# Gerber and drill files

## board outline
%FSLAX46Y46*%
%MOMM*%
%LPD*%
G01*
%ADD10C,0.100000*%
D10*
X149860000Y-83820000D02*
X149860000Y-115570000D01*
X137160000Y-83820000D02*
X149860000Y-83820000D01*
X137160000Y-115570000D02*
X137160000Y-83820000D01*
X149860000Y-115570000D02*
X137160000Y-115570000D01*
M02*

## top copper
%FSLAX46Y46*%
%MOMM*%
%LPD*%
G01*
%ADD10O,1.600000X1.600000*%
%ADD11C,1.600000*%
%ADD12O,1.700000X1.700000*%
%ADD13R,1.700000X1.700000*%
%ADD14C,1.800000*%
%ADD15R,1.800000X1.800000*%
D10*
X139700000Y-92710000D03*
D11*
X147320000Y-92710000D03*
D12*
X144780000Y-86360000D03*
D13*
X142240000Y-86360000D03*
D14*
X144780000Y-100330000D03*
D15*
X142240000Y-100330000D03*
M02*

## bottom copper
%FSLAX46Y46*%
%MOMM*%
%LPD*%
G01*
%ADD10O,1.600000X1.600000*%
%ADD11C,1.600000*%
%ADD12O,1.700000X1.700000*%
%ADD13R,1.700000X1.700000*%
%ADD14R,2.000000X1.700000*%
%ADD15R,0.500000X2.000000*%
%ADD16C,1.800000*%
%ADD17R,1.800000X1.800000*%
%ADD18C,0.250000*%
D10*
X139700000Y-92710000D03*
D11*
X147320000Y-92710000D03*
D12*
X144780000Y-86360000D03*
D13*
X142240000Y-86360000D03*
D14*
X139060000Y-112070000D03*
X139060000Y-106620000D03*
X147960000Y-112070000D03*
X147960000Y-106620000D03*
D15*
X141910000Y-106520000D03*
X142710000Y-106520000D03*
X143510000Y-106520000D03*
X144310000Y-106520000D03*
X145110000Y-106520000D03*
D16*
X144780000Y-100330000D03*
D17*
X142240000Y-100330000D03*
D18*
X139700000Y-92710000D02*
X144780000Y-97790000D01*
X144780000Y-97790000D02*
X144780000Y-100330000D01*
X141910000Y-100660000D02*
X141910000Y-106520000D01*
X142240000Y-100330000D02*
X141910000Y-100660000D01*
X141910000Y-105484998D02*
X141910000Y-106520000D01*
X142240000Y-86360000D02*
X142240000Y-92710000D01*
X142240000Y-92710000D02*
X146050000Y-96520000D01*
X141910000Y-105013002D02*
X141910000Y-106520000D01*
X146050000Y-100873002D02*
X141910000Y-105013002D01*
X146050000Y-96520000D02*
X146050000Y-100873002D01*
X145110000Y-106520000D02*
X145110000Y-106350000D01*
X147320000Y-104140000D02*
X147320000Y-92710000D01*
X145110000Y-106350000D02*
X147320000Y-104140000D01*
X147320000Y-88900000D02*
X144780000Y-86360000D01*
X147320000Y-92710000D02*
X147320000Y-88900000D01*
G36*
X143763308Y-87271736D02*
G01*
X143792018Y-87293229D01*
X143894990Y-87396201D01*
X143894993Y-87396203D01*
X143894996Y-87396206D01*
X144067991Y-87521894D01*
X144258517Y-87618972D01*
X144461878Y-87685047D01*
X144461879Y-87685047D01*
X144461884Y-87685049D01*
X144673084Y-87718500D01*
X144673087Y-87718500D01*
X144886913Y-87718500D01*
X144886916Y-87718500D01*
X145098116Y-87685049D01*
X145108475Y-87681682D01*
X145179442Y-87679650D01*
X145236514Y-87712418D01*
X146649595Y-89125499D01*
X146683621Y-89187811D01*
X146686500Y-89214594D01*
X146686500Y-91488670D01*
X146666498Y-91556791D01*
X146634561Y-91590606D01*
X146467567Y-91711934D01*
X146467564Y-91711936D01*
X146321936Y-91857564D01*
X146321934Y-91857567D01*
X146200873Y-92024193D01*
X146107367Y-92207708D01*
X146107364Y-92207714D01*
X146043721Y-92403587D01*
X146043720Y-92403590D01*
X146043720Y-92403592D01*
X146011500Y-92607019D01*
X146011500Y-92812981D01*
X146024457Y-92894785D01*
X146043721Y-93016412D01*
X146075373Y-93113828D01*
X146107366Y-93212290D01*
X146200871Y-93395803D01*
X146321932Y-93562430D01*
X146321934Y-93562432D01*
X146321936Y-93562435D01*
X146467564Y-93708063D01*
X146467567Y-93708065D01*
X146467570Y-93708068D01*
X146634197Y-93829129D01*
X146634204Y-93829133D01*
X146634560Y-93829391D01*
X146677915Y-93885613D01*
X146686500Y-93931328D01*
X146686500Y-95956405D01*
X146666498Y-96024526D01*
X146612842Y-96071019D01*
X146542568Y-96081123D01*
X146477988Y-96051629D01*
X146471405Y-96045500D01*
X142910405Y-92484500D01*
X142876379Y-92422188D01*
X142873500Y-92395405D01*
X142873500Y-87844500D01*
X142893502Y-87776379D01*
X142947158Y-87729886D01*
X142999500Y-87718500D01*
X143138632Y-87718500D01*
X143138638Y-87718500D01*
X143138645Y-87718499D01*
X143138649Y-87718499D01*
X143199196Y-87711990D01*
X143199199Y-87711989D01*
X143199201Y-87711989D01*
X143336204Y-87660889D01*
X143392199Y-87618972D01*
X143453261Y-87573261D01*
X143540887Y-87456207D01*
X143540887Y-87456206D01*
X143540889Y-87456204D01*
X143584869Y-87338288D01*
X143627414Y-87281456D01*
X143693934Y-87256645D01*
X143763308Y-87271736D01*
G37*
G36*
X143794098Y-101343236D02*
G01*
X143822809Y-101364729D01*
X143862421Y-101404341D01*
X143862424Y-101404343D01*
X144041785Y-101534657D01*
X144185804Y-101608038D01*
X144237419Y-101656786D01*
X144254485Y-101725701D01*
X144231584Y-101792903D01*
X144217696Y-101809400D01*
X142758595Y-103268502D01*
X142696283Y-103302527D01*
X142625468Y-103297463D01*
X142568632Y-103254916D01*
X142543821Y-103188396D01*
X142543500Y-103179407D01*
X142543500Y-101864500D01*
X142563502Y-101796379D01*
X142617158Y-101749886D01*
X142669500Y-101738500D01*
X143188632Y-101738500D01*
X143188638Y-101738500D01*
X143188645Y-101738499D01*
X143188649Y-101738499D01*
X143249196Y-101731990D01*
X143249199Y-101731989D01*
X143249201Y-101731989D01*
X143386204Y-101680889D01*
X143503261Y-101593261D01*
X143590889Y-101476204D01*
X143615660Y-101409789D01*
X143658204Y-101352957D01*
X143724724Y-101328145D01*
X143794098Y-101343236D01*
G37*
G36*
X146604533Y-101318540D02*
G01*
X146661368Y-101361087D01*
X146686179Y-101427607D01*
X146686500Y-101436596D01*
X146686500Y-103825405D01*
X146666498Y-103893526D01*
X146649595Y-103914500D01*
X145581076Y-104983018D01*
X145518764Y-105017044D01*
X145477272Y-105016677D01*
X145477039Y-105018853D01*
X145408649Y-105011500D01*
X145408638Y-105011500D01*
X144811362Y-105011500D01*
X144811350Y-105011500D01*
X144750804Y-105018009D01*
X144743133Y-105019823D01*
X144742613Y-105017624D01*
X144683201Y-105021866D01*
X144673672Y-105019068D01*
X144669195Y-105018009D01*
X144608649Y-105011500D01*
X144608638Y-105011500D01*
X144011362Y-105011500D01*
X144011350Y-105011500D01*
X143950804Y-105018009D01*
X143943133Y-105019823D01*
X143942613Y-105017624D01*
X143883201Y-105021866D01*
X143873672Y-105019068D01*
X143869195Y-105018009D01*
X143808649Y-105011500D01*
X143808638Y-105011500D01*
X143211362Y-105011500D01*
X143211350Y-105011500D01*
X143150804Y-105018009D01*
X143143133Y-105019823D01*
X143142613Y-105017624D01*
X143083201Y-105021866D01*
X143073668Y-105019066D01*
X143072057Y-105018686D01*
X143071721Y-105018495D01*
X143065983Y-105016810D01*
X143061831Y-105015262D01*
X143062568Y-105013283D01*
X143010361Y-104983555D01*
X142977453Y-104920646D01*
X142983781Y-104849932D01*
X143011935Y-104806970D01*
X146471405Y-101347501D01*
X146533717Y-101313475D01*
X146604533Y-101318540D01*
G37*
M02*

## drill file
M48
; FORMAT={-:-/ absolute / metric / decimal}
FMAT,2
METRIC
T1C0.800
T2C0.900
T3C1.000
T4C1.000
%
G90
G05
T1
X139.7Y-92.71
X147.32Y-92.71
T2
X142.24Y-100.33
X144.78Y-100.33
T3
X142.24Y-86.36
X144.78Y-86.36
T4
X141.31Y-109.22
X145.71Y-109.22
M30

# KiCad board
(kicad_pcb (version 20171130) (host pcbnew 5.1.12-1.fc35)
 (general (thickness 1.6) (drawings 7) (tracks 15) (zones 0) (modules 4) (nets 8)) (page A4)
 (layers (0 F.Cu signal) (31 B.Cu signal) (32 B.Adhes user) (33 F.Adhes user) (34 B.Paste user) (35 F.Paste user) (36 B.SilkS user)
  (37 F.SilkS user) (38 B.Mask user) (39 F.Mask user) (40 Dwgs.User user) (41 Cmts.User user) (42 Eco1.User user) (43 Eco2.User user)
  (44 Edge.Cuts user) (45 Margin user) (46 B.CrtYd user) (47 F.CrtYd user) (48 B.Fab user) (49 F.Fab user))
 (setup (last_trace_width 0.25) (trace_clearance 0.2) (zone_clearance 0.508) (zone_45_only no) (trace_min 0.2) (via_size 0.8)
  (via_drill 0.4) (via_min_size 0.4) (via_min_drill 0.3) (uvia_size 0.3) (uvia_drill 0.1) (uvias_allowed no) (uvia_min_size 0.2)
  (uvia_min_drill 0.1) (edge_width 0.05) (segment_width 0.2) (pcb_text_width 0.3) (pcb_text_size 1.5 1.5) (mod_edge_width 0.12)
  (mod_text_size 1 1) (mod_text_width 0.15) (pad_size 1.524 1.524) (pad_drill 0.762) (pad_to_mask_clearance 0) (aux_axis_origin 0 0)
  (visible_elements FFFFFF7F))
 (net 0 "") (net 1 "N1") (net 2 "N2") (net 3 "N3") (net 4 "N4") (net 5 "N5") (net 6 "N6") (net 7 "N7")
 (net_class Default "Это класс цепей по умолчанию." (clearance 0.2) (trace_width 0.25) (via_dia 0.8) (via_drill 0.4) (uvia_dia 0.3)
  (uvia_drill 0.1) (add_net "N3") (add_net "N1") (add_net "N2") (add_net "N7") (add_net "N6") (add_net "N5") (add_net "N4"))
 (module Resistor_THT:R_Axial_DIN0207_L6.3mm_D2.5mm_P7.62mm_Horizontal (layer F.Cu) (at 147.32 92.71 180)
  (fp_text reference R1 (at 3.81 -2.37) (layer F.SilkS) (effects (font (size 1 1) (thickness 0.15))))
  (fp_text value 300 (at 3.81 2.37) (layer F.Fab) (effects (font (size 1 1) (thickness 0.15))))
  (pad 2 thru_hole oval (at 7.62 0 180) (size 1.6 1.6) (drill 0.8) (layers *.Cu *.Mask) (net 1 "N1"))
  (pad 1 thru_hole circle (at 0 0 180) (size 1.6 1.6) (drill 0.8) (layers *.Cu *.Mask) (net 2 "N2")))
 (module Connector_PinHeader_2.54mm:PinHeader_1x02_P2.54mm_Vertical (layer F.Cu) (at 142.24 86.36 90)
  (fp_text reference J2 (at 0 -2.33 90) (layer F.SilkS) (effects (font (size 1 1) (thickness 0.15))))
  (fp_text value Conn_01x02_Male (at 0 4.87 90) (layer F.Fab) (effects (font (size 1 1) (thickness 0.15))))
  (pad 2 thru_hole oval (at 0 2.54 90) (size 1.7 1.7) (drill 1) (layers *.Cu *.Mask) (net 2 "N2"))
  (pad 1 thru_hole rect (at 0 0 90) (size 1.7 1.7) (drill 1) (layers *.Cu *.Mask) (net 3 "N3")))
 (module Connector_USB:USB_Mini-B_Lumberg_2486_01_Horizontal (layer B.Cu) (at 143.51 109.22 180)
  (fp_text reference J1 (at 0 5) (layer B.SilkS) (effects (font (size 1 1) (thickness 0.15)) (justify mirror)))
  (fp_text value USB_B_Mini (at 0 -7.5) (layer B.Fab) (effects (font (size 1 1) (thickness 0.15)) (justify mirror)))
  (pad "" np_thru_hole circle (at 2.2 0 180) (size 1 1) (drill 1) (layers *.Cu *.Mask))
  (pad "" np_thru_hole circle (at -2.2 0 180) (size 1 1) (drill 1) (layers *.Cu *.Mask))
  (pad 6 smd rect (at 4.45 -2.85 180) (size 2 1.7) (layers B.Cu B.Paste B.Mask) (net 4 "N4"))
  (pad 6 smd rect (at 4.45 2.6 180) (size 2 1.7) (layers B.Cu B.Paste B.Mask) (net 4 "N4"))
  (pad 6 smd rect (at -4.45 -2.85 180) (size 2 1.7) (layers B.Cu B.Paste B.Mask) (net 4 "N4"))
  (pad 6 smd rect (at -4.45 2.6 180) (size 2 1.7) (layers B.Cu B.Paste B.Mask) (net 4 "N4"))
  (pad 5 smd rect (at 1.6 2.7 180) (size 0.5 2) (layers B.Cu B.Paste B.Mask) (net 3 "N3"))
  (pad 4 smd rect (at 0.8 2.7 180) (size 0.5 2) (layers B.Cu B.Paste B.Mask) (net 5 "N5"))
  (pad 3 smd rect (at 0 2.7 180) (size 0.5 2) (layers B.Cu B.Paste B.Mask) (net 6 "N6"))
  (pad 2 smd rect (at -0.8 2.7 180) (size 0.5 2) (layers B.Cu B.Paste B.Mask) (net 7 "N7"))
  (pad 1 smd rect (at -1.6 2.7 180) (size 0.5 2) (layers B.Cu B.Paste B.Mask) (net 2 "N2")))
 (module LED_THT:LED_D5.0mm (layer F.Cu) (at 142.24 100.33)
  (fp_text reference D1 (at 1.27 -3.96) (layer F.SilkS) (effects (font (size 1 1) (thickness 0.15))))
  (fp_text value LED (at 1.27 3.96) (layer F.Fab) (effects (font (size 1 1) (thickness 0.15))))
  (pad 2 thru_hole circle (at 2.54 0) (size 1.8 1.8) (drill 0.9) (layers *.Cu *.Mask) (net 1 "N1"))
  (pad 1 thru_hole rect (at 0 0) (size 1.8 1.8) (drill 0.9) (layers *.Cu *.Mask) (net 3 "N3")))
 (gr_line (start 149.86 83.82) (end 149.86 115.57) (layer Edge.Cuts) (width 0.1))
 (gr_line (start 137.16 83.82) (end 149.86 83.82) (layer Edge.Cuts) (width 0.1))
 (gr_line (start 137.16 115.57) (end 137.16 83.82) (layer Edge.Cuts) (width 0.1))
 (gr_line (start 149.86 115.57) (end 137.16 115.57) (layer Edge.Cuts) (width 0.1))
 (segment (start 139.7 92.71) (end 144.78 97.79) (width 0.25) (layer B.Cu) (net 1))
 (segment (start 144.78 97.79) (end 144.78 100.33) (width 0.25) (layer B.Cu) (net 1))
 (segment (start 141.91 100.66) (end 141.91 106.52) (width 0.25) (layer B.Cu) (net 3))
 (segment (start 142.24 100.33) (end 141.91 100.66) (width 0.25) (layer B.Cu) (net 3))
 (segment (start 141.91 105.484998) (end 141.91 106.52) (width 0.25) (layer B.Cu) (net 3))
 (segment (start 142.24 86.36) (end 142.24 92.71) (width 0.25) (layer B.Cu) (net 3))
 (segment (start 142.24 92.71) (end 146.05 96.52) (width 0.25) (layer B.Cu) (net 3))
 (segment (start 141.91 105.013002) (end 141.91 106.52) (width 0.25) (layer B.Cu) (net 3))
 (segment (start 146.05 100.873002) (end 141.91 105.013002) (width 0.25) (layer B.Cu) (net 3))
 (segment (start 146.05 96.52) (end 146.05 100.873002) (width 0.25) (layer B.Cu) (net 3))
 (segment (start 145.11 106.52) (end 145.11 106.35) (width 0.25) (layer B.Cu) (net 2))
 (segment (start 147.32 104.14) (end 147.32 92.71) (width 0.25) (layer B.Cu) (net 2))
 (segment (start 145.11 106.35) (end 147.32 104.14) (width 0.25) (layer B.Cu) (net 2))
 (segment (start 147.32 88.9) (end 144.78 86.36) (width 0.25) (layer B.Cu) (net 2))
 (segment (start 147.32 92.71) (end 147.32 88.9) (width 0.25) (layer B.Cu) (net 2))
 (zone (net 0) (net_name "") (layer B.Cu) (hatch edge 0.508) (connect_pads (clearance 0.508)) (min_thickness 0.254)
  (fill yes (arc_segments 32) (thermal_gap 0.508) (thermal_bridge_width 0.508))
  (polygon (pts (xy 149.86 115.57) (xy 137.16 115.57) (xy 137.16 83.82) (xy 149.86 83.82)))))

